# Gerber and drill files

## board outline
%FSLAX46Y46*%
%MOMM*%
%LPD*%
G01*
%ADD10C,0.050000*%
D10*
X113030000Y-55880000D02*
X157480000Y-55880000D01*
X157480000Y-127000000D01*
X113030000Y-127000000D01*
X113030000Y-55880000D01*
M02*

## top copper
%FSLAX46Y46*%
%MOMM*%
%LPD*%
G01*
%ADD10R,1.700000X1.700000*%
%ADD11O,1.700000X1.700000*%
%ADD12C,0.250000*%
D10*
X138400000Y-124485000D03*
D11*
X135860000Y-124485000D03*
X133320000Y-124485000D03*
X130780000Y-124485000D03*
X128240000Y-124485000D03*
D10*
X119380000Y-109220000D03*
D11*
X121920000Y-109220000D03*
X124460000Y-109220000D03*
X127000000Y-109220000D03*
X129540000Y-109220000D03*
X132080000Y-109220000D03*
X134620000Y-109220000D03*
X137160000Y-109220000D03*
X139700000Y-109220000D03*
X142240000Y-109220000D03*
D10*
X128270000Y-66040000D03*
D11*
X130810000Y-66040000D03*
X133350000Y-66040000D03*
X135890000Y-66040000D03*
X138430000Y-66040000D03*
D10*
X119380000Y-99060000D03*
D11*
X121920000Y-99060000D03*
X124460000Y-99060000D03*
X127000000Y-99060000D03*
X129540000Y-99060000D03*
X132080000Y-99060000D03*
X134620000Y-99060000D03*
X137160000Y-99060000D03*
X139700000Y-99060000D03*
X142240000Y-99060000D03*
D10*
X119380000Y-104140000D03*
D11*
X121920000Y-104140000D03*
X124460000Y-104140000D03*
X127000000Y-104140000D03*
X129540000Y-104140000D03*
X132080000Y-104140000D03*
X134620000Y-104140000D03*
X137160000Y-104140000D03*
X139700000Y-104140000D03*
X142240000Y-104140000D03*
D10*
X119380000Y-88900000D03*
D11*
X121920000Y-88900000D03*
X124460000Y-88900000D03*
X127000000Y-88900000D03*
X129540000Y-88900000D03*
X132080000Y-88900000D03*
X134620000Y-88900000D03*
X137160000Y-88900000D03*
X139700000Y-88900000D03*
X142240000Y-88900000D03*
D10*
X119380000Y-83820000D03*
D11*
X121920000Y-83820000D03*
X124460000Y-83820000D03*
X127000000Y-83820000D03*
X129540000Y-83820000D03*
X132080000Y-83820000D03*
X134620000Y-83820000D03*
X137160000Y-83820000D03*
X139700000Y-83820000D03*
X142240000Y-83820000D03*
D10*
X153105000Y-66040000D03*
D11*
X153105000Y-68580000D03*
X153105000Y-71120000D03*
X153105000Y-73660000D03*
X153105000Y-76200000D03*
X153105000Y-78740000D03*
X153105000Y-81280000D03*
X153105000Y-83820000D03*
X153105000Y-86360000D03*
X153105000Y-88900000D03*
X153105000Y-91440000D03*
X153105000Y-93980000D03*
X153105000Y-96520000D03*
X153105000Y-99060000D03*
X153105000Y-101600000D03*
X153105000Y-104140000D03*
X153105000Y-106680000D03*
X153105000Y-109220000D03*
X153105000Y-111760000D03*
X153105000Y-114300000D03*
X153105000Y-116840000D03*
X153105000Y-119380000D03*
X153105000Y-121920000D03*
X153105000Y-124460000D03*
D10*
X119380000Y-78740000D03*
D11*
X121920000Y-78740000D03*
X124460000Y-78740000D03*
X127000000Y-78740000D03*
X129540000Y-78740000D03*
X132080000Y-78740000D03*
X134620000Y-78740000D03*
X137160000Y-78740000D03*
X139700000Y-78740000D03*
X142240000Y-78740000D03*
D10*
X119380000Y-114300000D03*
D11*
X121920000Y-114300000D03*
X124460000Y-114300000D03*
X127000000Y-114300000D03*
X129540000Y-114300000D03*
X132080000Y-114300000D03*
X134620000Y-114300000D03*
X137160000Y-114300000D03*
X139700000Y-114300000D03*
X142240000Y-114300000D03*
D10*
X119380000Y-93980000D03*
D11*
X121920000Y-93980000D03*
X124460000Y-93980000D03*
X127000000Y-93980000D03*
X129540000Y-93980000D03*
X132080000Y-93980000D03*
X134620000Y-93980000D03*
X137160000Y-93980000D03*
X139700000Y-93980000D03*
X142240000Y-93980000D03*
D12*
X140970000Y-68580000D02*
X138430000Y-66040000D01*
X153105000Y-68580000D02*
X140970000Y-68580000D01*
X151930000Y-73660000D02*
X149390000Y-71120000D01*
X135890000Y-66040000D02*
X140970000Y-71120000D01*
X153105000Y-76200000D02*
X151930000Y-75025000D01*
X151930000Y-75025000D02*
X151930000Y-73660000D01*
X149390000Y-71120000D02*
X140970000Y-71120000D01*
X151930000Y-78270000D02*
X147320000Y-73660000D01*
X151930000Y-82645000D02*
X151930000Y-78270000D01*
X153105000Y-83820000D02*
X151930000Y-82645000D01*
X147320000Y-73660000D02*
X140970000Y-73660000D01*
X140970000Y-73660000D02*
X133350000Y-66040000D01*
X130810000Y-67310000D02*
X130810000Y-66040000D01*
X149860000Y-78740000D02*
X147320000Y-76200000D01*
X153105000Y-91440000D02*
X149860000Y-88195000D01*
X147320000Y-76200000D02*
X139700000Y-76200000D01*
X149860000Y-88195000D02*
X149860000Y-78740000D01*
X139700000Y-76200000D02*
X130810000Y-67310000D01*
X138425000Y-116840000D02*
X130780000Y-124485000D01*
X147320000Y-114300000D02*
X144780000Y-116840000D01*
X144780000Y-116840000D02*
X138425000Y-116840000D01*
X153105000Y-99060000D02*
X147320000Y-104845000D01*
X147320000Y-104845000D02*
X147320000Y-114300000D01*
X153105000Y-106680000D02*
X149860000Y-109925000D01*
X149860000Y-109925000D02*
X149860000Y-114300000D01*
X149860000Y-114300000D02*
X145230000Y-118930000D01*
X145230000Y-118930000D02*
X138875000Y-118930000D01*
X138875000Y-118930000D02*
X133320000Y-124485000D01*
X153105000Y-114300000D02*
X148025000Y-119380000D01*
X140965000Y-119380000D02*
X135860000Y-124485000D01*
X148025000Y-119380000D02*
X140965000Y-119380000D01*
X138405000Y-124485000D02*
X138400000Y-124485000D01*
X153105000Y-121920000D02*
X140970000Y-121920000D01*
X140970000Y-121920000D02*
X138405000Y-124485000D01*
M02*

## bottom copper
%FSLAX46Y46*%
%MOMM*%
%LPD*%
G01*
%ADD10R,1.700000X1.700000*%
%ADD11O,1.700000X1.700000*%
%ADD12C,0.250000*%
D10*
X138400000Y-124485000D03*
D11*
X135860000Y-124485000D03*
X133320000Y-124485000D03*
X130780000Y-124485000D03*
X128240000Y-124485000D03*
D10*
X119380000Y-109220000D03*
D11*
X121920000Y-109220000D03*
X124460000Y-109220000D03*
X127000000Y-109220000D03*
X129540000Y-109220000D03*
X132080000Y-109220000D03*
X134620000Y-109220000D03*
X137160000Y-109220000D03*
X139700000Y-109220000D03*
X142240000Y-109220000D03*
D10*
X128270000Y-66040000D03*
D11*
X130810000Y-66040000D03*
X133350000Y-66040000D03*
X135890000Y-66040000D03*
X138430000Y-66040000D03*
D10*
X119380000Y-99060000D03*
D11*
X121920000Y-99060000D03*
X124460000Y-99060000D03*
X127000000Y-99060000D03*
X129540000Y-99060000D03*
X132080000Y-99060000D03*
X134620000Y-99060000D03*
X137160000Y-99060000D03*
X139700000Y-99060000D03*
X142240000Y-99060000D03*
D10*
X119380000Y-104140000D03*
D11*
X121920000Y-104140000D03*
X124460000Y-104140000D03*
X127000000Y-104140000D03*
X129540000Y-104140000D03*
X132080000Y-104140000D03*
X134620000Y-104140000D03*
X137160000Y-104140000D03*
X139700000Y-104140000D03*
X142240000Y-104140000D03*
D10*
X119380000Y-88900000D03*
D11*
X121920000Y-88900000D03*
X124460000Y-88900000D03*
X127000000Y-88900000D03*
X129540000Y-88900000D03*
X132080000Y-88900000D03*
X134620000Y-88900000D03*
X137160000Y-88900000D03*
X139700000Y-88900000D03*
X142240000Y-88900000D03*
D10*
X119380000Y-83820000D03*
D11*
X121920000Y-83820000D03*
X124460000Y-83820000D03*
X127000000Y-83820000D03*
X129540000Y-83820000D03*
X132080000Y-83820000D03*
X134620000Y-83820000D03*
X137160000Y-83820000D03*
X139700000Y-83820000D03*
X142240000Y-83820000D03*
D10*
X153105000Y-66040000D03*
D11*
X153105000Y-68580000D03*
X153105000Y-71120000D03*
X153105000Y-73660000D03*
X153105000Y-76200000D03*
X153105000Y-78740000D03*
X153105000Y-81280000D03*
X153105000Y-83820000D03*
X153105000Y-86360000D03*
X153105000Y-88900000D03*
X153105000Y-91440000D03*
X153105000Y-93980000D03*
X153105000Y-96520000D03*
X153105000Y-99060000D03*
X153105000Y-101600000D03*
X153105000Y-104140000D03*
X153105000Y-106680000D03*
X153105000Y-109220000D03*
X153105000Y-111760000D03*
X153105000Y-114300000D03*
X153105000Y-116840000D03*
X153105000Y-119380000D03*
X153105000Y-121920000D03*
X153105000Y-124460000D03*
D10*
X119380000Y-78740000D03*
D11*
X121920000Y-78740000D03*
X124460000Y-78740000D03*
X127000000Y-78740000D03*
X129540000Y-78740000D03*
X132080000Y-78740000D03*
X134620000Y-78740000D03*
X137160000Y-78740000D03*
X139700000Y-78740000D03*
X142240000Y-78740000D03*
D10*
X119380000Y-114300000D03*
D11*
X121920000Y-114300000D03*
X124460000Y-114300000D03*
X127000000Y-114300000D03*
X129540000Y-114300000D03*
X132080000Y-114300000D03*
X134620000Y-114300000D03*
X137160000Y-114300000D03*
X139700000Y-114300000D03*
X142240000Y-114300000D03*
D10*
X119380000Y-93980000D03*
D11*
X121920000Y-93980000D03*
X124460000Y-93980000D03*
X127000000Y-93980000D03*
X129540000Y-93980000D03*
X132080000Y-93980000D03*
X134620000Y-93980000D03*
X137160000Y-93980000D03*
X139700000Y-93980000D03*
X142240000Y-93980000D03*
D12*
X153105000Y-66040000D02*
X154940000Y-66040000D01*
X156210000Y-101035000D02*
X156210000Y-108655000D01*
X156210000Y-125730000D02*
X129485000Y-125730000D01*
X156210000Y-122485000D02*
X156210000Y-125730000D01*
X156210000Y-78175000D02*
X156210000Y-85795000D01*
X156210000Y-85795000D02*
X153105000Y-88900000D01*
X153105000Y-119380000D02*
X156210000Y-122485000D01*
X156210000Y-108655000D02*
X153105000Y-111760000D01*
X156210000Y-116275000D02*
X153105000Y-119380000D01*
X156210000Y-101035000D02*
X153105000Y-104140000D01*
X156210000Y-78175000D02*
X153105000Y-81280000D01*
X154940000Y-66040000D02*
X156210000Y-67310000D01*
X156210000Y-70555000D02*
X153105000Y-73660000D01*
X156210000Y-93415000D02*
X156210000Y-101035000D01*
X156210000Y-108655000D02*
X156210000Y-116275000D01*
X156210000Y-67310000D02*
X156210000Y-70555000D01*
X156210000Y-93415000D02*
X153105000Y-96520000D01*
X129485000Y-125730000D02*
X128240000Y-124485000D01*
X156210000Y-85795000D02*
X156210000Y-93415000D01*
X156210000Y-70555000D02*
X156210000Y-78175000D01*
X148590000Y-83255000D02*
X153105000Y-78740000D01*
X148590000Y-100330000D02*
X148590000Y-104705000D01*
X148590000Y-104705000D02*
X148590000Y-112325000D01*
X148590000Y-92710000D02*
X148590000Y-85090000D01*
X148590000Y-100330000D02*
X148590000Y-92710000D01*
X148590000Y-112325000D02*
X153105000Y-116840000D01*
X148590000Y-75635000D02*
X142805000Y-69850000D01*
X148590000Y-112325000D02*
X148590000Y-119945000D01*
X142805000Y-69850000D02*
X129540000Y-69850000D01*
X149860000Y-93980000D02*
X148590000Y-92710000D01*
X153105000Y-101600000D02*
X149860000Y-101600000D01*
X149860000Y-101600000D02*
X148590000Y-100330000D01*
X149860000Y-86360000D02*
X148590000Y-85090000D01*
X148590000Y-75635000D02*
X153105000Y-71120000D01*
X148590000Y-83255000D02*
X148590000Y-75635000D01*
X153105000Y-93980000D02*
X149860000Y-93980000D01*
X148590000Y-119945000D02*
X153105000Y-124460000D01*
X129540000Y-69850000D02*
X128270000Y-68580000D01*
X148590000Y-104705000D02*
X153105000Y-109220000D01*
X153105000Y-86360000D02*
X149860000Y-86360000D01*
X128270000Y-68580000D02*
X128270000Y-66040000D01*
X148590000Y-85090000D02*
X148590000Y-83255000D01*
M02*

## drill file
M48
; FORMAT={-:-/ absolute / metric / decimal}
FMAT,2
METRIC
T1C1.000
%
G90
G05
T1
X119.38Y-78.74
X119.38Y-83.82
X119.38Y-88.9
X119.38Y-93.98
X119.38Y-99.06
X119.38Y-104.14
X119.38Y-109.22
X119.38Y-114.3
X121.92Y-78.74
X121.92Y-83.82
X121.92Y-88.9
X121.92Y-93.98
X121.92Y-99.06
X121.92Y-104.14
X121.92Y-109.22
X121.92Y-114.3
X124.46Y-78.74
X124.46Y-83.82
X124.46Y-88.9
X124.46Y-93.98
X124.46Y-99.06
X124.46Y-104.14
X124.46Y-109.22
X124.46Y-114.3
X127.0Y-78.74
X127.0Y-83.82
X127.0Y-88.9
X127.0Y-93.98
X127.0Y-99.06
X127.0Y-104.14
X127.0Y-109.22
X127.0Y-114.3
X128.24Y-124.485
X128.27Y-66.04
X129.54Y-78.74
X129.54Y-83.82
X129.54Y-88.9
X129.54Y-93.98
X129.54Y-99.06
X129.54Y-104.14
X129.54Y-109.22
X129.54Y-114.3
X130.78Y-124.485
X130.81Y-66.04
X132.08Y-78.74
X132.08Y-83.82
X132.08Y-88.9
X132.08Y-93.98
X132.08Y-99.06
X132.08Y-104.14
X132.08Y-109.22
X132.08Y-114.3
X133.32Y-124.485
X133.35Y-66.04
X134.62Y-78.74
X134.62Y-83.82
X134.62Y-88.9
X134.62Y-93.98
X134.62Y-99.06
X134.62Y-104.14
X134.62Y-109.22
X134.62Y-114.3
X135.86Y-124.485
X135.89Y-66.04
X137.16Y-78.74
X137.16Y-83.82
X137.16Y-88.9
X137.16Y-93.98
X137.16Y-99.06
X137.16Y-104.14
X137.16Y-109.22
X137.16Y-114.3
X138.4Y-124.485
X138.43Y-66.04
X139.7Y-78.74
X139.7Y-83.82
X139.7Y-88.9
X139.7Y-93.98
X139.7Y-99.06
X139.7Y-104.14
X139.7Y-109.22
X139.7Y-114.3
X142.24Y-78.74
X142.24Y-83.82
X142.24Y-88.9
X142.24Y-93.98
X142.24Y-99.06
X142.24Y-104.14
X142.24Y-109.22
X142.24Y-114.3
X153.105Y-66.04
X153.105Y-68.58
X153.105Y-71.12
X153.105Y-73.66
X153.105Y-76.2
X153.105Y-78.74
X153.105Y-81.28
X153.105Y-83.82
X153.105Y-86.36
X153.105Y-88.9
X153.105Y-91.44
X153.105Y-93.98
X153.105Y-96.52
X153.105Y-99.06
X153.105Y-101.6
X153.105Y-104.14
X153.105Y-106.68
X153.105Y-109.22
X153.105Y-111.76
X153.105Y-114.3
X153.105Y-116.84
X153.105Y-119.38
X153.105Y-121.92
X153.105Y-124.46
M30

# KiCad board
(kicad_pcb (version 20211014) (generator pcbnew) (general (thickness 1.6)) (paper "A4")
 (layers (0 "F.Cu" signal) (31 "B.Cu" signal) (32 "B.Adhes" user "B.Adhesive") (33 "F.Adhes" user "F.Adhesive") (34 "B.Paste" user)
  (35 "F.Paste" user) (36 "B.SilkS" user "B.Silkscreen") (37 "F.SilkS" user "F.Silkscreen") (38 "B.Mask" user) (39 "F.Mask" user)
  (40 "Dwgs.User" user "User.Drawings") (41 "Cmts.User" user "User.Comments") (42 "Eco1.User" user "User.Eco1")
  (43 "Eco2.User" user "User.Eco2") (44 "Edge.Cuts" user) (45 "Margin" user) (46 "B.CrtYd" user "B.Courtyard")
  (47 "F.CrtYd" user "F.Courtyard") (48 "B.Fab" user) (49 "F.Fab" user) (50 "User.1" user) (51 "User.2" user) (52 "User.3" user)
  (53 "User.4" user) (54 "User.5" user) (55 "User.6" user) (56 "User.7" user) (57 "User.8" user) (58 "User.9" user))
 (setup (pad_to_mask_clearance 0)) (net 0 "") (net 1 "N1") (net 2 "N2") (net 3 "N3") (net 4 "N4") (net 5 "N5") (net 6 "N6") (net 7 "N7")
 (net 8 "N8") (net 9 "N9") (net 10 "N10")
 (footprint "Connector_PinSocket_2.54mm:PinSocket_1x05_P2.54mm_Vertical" (layer "F.Cu") (at 138.4 124.485 -90)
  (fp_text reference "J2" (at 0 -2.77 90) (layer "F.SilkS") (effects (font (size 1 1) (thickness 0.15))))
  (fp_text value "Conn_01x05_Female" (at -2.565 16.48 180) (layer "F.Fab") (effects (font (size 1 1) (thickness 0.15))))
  (pad "1" thru_hole rect (at 0 0 270) (size 1.7 1.7) (drill 1) (layers *.Cu *.Mask) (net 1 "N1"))
  (pad "2" thru_hole oval (at 0 2.54 270) (size 1.7 1.7) (drill 1) (layers *.Cu *.Mask) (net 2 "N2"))
  (pad "3" thru_hole oval (at 0 5.08 270) (size 1.7 1.7) (drill 1) (layers *.Cu *.Mask) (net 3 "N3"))
  (pad "4" thru_hole oval (at 0 7.62 270) (size 1.7 1.7) (drill 1) (layers *.Cu *.Mask) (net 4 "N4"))
  (pad "5" thru_hole oval (at 0 10.16 270) (size 1.7 1.7) (drill 1) (layers *.Cu *.Mask) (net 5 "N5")))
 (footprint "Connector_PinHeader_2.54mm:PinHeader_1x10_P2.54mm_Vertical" (layer "F.Cu") (at 119.38 109.22 90)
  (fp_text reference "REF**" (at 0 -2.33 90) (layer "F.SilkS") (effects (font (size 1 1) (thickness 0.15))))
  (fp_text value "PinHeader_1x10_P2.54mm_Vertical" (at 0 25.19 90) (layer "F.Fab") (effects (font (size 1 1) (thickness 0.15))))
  (pad "1" thru_hole rect (at 0 0 90) (size 1.7 1.7) (drill 1) (layers *.Cu *.Mask))
  (pad "2" thru_hole oval (at 0 2.54 90) (size 1.7 1.7) (drill 1) (layers *.Cu *.Mask))
  (pad "3" thru_hole oval (at 0 5.08 90) (size 1.7 1.7) (drill 1) (layers *.Cu *.Mask))
  (pad "4" thru_hole oval (at 0 7.62 90) (size 1.7 1.7) (drill 1) (layers *.Cu *.Mask))
  (pad "5" thru_hole oval (at 0 10.16 90) (size 1.7 1.7) (drill 1) (layers *.Cu *.Mask))
  (pad "6" thru_hole oval (at 0 12.7 90) (size 1.7 1.7) (drill 1) (layers *.Cu *.Mask))
  (pad "7" thru_hole oval (at 0 15.24 90) (size 1.7 1.7) (drill 1) (layers *.Cu *.Mask))
  (pad "8" thru_hole oval (at 0 17.78 90) (size 1.7 1.7) (drill 1) (layers *.Cu *.Mask))
  (pad "9" thru_hole oval (at 0 20.32 90) (size 1.7 1.7) (drill 1) (layers *.Cu *.Mask))
  (pad "10" thru_hole oval (at 0 22.86 90) (size 1.7 1.7) (drill 1) (layers *.Cu *.Mask)))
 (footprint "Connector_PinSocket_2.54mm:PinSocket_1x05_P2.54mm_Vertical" (layer "F.Cu") (at 128.27 66.04 90)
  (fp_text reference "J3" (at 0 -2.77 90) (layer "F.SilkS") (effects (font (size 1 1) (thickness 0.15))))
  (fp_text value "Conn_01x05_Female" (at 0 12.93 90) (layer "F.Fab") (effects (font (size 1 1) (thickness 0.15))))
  (pad "1" thru_hole rect (at 0 0 90) (size 1.7 1.7) (drill 1) (layers *.Cu *.Mask) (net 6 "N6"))
  (pad "2" thru_hole oval (at 0 2.54 90) (size 1.7 1.7) (drill 1) (layers *.Cu *.Mask) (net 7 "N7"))
  (pad "3" thru_hole oval (at 0 5.08 90) (size 1.7 1.7) (drill 1) (layers *.Cu *.Mask) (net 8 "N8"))
  (pad "4" thru_hole oval (at 0 7.62 90) (size 1.7 1.7) (drill 1) (layers *.Cu *.Mask) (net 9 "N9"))
  (pad "5" thru_hole oval (at 0 10.16 90) (size 1.7 1.7) (drill 1) (layers *.Cu *.Mask) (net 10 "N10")))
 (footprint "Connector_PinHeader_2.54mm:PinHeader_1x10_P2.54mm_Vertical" (layer "F.Cu") (at 119.38 99.06 90)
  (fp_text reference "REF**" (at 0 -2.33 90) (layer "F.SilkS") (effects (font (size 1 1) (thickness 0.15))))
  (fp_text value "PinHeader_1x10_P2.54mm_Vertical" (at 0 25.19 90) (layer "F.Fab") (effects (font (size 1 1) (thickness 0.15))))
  (pad "1" thru_hole rect (at 0 0 90) (size 1.7 1.7) (drill 1) (layers *.Cu *.Mask))
  (pad "2" thru_hole oval (at 0 2.54 90) (size 1.7 1.7) (drill 1) (layers *.Cu *.Mask))
  (pad "3" thru_hole oval (at 0 5.08 90) (size 1.7 1.7) (drill 1) (layers *.Cu *.Mask))
  (pad "4" thru_hole oval (at 0 7.62 90) (size 1.7 1.7) (drill 1) (layers *.Cu *.Mask))
  (pad "5" thru_hole oval (at 0 10.16 90) (size 1.7 1.7) (drill 1) (layers *.Cu *.Mask))
  (pad "6" thru_hole oval (at 0 12.7 90) (size 1.7 1.7) (drill 1) (layers *.Cu *.Mask))
  (pad "7" thru_hole oval (at 0 15.24 90) (size 1.7 1.7) (drill 1) (layers *.Cu *.Mask))
  (pad "8" thru_hole oval (at 0 17.78 90) (size 1.7 1.7) (drill 1) (layers *.Cu *.Mask))
  (pad "9" thru_hole oval (at 0 20.32 90) (size 1.7 1.7) (drill 1) (layers *.Cu *.Mask))
  (pad "10" thru_hole oval (at 0 22.86 90) (size 1.7 1.7) (drill 1) (layers *.Cu *.Mask)))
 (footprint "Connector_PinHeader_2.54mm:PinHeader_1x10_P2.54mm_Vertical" (layer "F.Cu") (at 119.38 104.14 90)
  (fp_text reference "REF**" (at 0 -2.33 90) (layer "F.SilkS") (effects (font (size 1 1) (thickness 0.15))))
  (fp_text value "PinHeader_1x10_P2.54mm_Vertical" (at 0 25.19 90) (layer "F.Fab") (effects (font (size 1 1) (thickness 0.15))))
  (pad "1" thru_hole rect (at 0 0 90) (size 1.7 1.7) (drill 1) (layers *.Cu *.Mask))
  (pad "2" thru_hole oval (at 0 2.54 90) (size 1.7 1.7) (drill 1) (layers *.Cu *.Mask))
  (pad "3" thru_hole oval (at 0 5.08 90) (size 1.7 1.7) (drill 1) (layers *.Cu *.Mask))
  (pad "4" thru_hole oval (at 0 7.62 90) (size 1.7 1.7) (drill 1) (layers *.Cu *.Mask))
  (pad "5" thru_hole oval (at 0 10.16 90) (size 1.7 1.7) (drill 1) (layers *.Cu *.Mask))
  (pad "6" thru_hole oval (at 0 12.7 90) (size 1.7 1.7) (drill 1) (layers *.Cu *.Mask))
  (pad "7" thru_hole oval (at 0 15.24 90) (size 1.7 1.7) (drill 1) (layers *.Cu *.Mask))
  (pad "8" thru_hole oval (at 0 17.78 90) (size 1.7 1.7) (drill 1) (layers *.Cu *.Mask))
  (pad "9" thru_hole oval (at 0 20.32 90) (size 1.7 1.7) (drill 1) (layers *.Cu *.Mask))
  (pad "10" thru_hole oval (at 0 22.86 90) (size 1.7 1.7) (drill 1) (layers *.Cu *.Mask)))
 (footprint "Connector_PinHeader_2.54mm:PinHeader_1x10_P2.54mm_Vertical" (layer "F.Cu") (at 119.38 88.9 90)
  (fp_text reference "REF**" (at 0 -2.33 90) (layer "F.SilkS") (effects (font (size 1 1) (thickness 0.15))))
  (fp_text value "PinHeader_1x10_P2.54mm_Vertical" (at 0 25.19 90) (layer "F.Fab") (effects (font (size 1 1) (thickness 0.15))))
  (pad "1" thru_hole rect (at 0 0 90) (size 1.7 1.7) (drill 1) (layers *.Cu *.Mask))
  (pad "2" thru_hole oval (at 0 2.54 90) (size 1.7 1.7) (drill 1) (layers *.Cu *.Mask))
  (pad "3" thru_hole oval (at 0 5.08 90) (size 1.7 1.7) (drill 1) (layers *.Cu *.Mask))
  (pad "4" thru_hole oval (at 0 7.62 90) (size 1.7 1.7) (drill 1) (layers *.Cu *.Mask))
  (pad "5" thru_hole oval (at 0 10.16 90) (size 1.7 1.7) (drill 1) (layers *.Cu *.Mask))
  (pad "6" thru_hole oval (at 0 12.7 90) (size 1.7 1.7) (drill 1) (layers *.Cu *.Mask))
  (pad "7" thru_hole oval (at 0 15.24 90) (size 1.7 1.7) (drill 1) (layers *.Cu *.Mask))
  (pad "8" thru_hole oval (at 0 17.78 90) (size 1.7 1.7) (drill 1) (layers *.Cu *.Mask))
  (pad "9" thru_hole oval (at 0 20.32 90) (size 1.7 1.7) (drill 1) (layers *.Cu *.Mask))
  (pad "10" thru_hole oval (at 0 22.86 90) (size 1.7 1.7) (drill 1) (layers *.Cu *.Mask)))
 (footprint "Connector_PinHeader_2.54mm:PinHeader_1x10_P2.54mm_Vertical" (layer "F.Cu") (at 119.38 83.82 90)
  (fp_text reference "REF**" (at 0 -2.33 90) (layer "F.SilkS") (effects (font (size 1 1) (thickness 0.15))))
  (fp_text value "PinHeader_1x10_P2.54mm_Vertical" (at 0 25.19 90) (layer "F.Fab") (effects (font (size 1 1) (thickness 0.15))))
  (pad "1" thru_hole rect (at 0 0 90) (size 1.7 1.7) (drill 1) (layers *.Cu *.Mask))
  (pad "2" thru_hole oval (at 0 2.54 90) (size 1.7 1.7) (drill 1) (layers *.Cu *.Mask))
  (pad "3" thru_hole oval (at 0 5.08 90) (size 1.7 1.7) (drill 1) (layers *.Cu *.Mask))
  (pad "4" thru_hole oval (at 0 7.62 90) (size 1.7 1.7) (drill 1) (layers *.Cu *.Mask))
  (pad "5" thru_hole oval (at 0 10.16 90) (size 1.7 1.7) (drill 1) (layers *.Cu *.Mask))
  (pad "6" thru_hole oval (at 0 12.7 90) (size 1.7 1.7) (drill 1) (layers *.Cu *.Mask))
  (pad "7" thru_hole oval (at 0 15.24 90) (size 1.7 1.7) (drill 1) (layers *.Cu *.Mask))
  (pad "8" thru_hole oval (at 0 17.78 90) (size 1.7 1.7) (drill 1) (layers *.Cu *.Mask))
  (pad "9" thru_hole oval (at 0 20.32 90) (size 1.7 1.7) (drill 1) (layers *.Cu *.Mask))
  (pad "10" thru_hole oval (at 0 22.86 90) (size 1.7 1.7) (drill 1) (layers *.Cu *.Mask)))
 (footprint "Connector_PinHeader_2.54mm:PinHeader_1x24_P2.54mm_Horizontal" (layer "F.Cu") (at 153.105 66.04)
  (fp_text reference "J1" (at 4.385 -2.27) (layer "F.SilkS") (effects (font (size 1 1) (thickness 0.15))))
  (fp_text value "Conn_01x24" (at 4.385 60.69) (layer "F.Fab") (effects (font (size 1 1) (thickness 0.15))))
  (pad "1" thru_hole rect (at 0 0) (size 1.7 1.7) (drill 1) (layers *.Cu *.Mask) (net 5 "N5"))
  (pad "2" thru_hole oval (at 0 2.54) (size 1.7 1.7) (drill 1) (layers *.Cu *.Mask) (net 10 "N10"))
  (pad "3" thru_hole oval (at 0 5.08) (size 1.7 1.7) (drill 1) (layers *.Cu *.Mask) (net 6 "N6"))
  (pad "4" thru_hole oval (at 0 7.62) (size 1.7 1.7) (drill 1) (layers *.Cu *.Mask) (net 5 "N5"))
  (pad "5" thru_hole oval (at 0 10.16) (size 1.7 1.7) (drill 1) (layers *.Cu *.Mask) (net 9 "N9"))
  (pad "6" thru_hole oval (at 0 12.7) (size 1.7 1.7) (drill 1) (layers *.Cu *.Mask) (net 6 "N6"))
  (pad "7" thru_hole oval (at 0 15.24) (size 1.7 1.7) (drill 1) (layers *.Cu *.Mask) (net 5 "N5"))
  (pad "8" thru_hole oval (at 0 17.78) (size 1.7 1.7) (drill 1) (layers *.Cu *.Mask) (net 8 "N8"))
  (pad "9" thru_hole oval (at 0 20.32) (size 1.7 1.7) (drill 1) (layers *.Cu *.Mask) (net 6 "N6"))
  (pad "10" thru_hole oval (at 0 22.86) (size 1.7 1.7) (drill 1) (layers *.Cu *.Mask) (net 5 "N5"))
  (pad "11" thru_hole oval (at 0 25.4) (size 1.7 1.7) (drill 1) (layers *.Cu *.Mask) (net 7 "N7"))
  (pad "12" thru_hole oval (at 0 27.94) (size 1.7 1.7) (drill 1) (layers *.Cu *.Mask) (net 6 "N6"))
  (pad "13" thru_hole oval (at 0 30.48) (size 1.7 1.7) (drill 1) (layers *.Cu *.Mask) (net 5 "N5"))
  (pad "14" thru_hole oval (at 0 33.02) (size 1.7 1.7) (drill 1) (layers *.Cu *.Mask) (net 4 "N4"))
  (pad "15" thru_hole oval (at 0 35.56) (size 1.7 1.7) (drill 1) (layers *.Cu *.Mask) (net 6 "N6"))
  (pad "16" thru_hole oval (at 0 38.1) (size 1.7 1.7) (drill 1) (layers *.Cu *.Mask) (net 5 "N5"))
  (pad "17" thru_hole oval (at 0 40.64) (size 1.7 1.7) (drill 1) (layers *.Cu *.Mask) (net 3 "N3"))
  (pad "18" thru_hole oval (at 0 43.18) (size 1.7 1.7) (drill 1) (layers *.Cu *.Mask) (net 6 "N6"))
  (pad "19" thru_hole oval (at 0 45.72) (size 1.7 1.7) (drill 1) (layers *.Cu *.Mask) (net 5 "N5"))
  (pad "20" thru_hole oval (at 0 48.26) (size 1.7 1.7) (drill 1) (layers *.Cu *.Mask) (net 2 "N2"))
  (pad "21" thru_hole oval (at 0 50.8) (size 1.7 1.7) (drill 1) (layers *.Cu *.Mask) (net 6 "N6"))
  (pad "22" thru_hole oval (at 0 53.34) (size 1.7 1.7) (drill 1) (layers *.Cu *.Mask) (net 5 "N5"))
  (pad "23" thru_hole oval (at 0 55.88) (size 1.7 1.7) (drill 1) (layers *.Cu *.Mask) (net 1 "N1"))
  (pad "24" thru_hole oval (at 0 58.42) (size 1.7 1.7) (drill 1) (layers *.Cu *.Mask) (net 6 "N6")))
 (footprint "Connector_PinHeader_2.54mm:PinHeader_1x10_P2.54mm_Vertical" (layer "F.Cu") (at 119.38 78.74 90)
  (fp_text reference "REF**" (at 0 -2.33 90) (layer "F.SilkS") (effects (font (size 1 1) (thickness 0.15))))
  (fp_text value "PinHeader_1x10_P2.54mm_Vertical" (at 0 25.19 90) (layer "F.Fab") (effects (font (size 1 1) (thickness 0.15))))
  (pad "1" thru_hole rect (at 0 0 90) (size 1.7 1.7) (drill 1) (layers *.Cu *.Mask))
  (pad "2" thru_hole oval (at 0 2.54 90) (size 1.7 1.7) (drill 1) (layers *.Cu *.Mask))
  (pad "3" thru_hole oval (at 0 5.08 90) (size 1.7 1.7) (drill 1) (layers *.Cu *.Mask))
  (pad "4" thru_hole oval (at 0 7.62 90) (size 1.7 1.7) (drill 1) (layers *.Cu *.Mask))
  (pad "5" thru_hole oval (at 0 10.16 90) (size 1.7 1.7) (drill 1) (layers *.Cu *.Mask))
  (pad "6" thru_hole oval (at 0 12.7 90) (size 1.7 1.7) (drill 1) (layers *.Cu *.Mask))
  (pad "7" thru_hole oval (at 0 15.24 90) (size 1.7 1.7) (drill 1) (layers *.Cu *.Mask))
  (pad "8" thru_hole oval (at 0 17.78 90) (size 1.7 1.7) (drill 1) (layers *.Cu *.Mask))
  (pad "9" thru_hole oval (at 0 20.32 90) (size 1.7 1.7) (drill 1) (layers *.Cu *.Mask))
  (pad "10" thru_hole oval (at 0 22.86 90) (size 1.7 1.7) (drill 1) (layers *.Cu *.Mask)))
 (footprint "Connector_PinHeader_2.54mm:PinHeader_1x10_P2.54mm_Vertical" (layer "F.Cu") (at 119.38 114.3 90)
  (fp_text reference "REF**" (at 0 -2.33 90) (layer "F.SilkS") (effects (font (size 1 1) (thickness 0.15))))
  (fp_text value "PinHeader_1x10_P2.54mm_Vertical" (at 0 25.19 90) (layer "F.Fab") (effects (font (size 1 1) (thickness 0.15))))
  (pad "1" thru_hole rect (at 0 0 90) (size 1.7 1.7) (drill 1) (layers *.Cu *.Mask))
  (pad "2" thru_hole oval (at 0 2.54 90) (size 1.7 1.7) (drill 1) (layers *.Cu *.Mask))
  (pad "3" thru_hole oval (at 0 5.08 90) (size 1.7 1.7) (drill 1) (layers *.Cu *.Mask))
  (pad "4" thru_hole oval (at 0 7.62 90) (size 1.7 1.7) (drill 1) (layers *.Cu *.Mask))
  (pad "5" thru_hole oval (at 0 10.16 90) (size 1.7 1.7) (drill 1) (layers *.Cu *.Mask))
  (pad "6" thru_hole oval (at 0 12.7 90) (size 1.7 1.7) (drill 1) (layers *.Cu *.Mask))
  (pad "7" thru_hole oval (at 0 15.24 90) (size 1.7 1.7) (drill 1) (layers *.Cu *.Mask))
  (pad "8" thru_hole oval (at 0 17.78 90) (size 1.7 1.7) (drill 1) (layers *.Cu *.Mask))
  (pad "9" thru_hole oval (at 0 20.32 90) (size 1.7 1.7) (drill 1) (layers *.Cu *.Mask))
  (pad "10" thru_hole oval (at 0 22.86 90) (size 1.7 1.7) (drill 1) (layers *.Cu *.Mask)))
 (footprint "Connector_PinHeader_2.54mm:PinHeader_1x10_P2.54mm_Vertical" (layer "F.Cu") (at 119.38 93.98 90)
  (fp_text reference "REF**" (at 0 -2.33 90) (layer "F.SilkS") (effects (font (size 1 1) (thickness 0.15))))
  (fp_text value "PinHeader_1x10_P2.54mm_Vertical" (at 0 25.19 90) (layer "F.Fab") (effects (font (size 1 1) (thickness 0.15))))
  (pad "1" thru_hole rect (at 0 0 90) (size 1.7 1.7) (drill 1) (layers *.Cu *.Mask))
  (pad "2" thru_hole oval (at 0 2.54 90) (size 1.7 1.7) (drill 1) (layers *.Cu *.Mask))
  (pad "3" thru_hole oval (at 0 5.08 90) (size 1.7 1.7) (drill 1) (layers *.Cu *.Mask))
  (pad "4" thru_hole oval (at 0 7.62 90) (size 1.7 1.7) (drill 1) (layers *.Cu *.Mask))
  (pad "5" thru_hole oval (at 0 10.16 90) (size 1.7 1.7) (drill 1) (layers *.Cu *.Mask))
  (pad "6" thru_hole oval (at 0 12.7 90) (size 1.7 1.7) (drill 1) (layers *.Cu *.Mask))
  (pad "7" thru_hole oval (at 0 15.24 90) (size 1.7 1.7) (drill 1) (layers *.Cu *.Mask))
  (pad "8" thru_hole oval (at 0 17.78 90) (size 1.7 1.7) (drill 1) (layers *.Cu *.Mask))
  (pad "9" thru_hole oval (at 0 20.32 90) (size 1.7 1.7) (drill 1) (layers *.Cu *.Mask))
  (pad "10" thru_hole oval (at 0 22.86 90) (size 1.7 1.7) (drill 1) (layers *.Cu *.Mask)))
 (gr_rect (start 157.48 127) (end 113.03 55.88) (layer "Edge.Cuts") (width 0.05) (fill none))
 (segment (start 153.105 66.04) (end 154.94 66.04) (width 0.25) (layer "B.Cu") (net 5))
 (segment (start 156.21 101.035) (end 156.21 108.655) (width 0.25) (layer "B.Cu") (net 5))
 (segment (start 156.21 125.73) (end 129.485 125.73) (width 0.25) (layer "B.Cu") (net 5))
 (segment (start 156.21 122.485) (end 156.21 125.73) (width 0.25) (layer "B.Cu") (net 5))
 (segment (start 156.21 78.175) (end 156.21 85.795) (width 0.25) (layer "B.Cu") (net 5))
 (segment (start 156.21 85.795) (end 153.105 88.9) (width 0.25) (layer "B.Cu") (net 5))
 (segment (start 153.105 119.38) (end 156.21 122.485) (width 0.25) (layer "B.Cu") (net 5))
 (segment (start 156.21 108.655) (end 153.105 111.76) (width 0.25) (layer "B.Cu") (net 5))
 (segment (start 156.21 116.275) (end 153.105 119.38) (width 0.25) (layer "B.Cu") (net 5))
 (segment (start 156.21 101.035) (end 153.105 104.14) (width 0.25) (layer "B.Cu") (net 5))
 (segment (start 156.21 78.175) (end 153.105 81.28) (width 0.25) (layer "B.Cu") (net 5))
 (segment (start 154.94 66.04) (end 156.21 67.31) (width 0.25) (layer "B.Cu") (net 5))
 (segment (start 156.21 70.555) (end 153.105 73.66) (width 0.25) (layer "B.Cu") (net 5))
 (segment (start 156.21 93.415) (end 156.21 101.035) (width 0.25) (layer "B.Cu") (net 5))
 (segment (start 156.21 108.655) (end 156.21 116.275) (width 0.25) (layer "B.Cu") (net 5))
 (segment (start 156.21 67.31) (end 156.21 70.555) (width 0.25) (layer "B.Cu") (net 5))
 (segment (start 156.21 93.415) (end 153.105 96.52) (width 0.25) (layer "B.Cu") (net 5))
 (segment (start 129.485 125.73) (end 128.24 124.485) (width 0.25) (layer "B.Cu") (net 5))
 (segment (start 156.21 85.795) (end 156.21 93.415) (width 0.25) (layer "B.Cu") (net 5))
 (segment (start 156.21 70.555) (end 156.21 78.175) (width 0.25) (layer "B.Cu") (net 5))
 (segment (start 140.97 68.58) (end 138.43 66.04) (width 0.25) (layer "F.Cu") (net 10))
 (segment (start 153.105 68.58) (end 140.97 68.58) (width 0.25) (layer "F.Cu") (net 10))
 (segment (start 151.93 73.66) (end 149.39 71.12) (width 0.25) (layer "F.Cu") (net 9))
 (segment (start 135.89 66.04) (end 140.97 71.12) (width 0.25) (layer "F.Cu") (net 9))
 (segment (start 153.105 76.2) (end 151.93 75.025) (width 0.25) (layer "F.Cu") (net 9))
 (segment (start 151.93 75.025) (end 151.93 73.66) (width 0.25) (layer "F.Cu") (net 9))
 (segment (start 149.39 71.12) (end 140.97 71.12) (width 0.25) (layer "F.Cu") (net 9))
 (segment (start 151.93 78.27) (end 147.32 73.66) (width 0.25) (layer "F.Cu") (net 8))
 (segment (start 151.93 82.645) (end 151.93 78.27) (width 0.25) (layer "F.Cu") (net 8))
 (segment (start 153.105 83.82) (end 151.93 82.645) (width 0.25) (layer "F.Cu") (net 8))
 (segment (start 147.32 73.66) (end 140.97 73.66) (width 0.25) (layer "F.Cu") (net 8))
 (segment (start 140.97 73.66) (end 133.35 66.04) (width 0.25) (layer "F.Cu") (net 8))
 (segment (start 130.81 67.31) (end 130.81 66.04) (width 0.25) (layer "F.Cu") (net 7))
 (segment (start 149.86 78.74) (end 147.32 76.2) (width 0.25) (layer "F.Cu") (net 7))
 (segment (start 153.105 91.44) (end 149.86 88.195) (width 0.25) (layer "F.Cu") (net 7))
 (segment (start 147.32 76.2) (end 139.7 76.2) (width 0.25) (layer "F.Cu") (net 7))
 (segment (start 149.86 88.195) (end 149.86 78.74) (width 0.25) (layer "F.Cu") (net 7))
 (segment (start 139.7 76.2) (end 130.81 67.31) (width 0.25) (layer "F.Cu") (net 7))
 (segment (start 148.59 83.255) (end 153.105 78.74) (width 0.25) (layer "B.Cu") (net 6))
 (segment (start 148.59 100.33) (end 148.59 104.705) (width 0.25) (layer "B.Cu") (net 6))
 (segment (start 148.59 104.705) (end 148.59 112.325) (width 0.25) (layer "B.Cu") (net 6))
 (segment (start 148.59 92.71) (end 148.59 85.09) (width 0.25) (layer "B.Cu") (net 6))
 (segment (start 148.59 100.33) (end 148.59 92.71) (width 0.25) (layer "B.Cu") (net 6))
 (segment (start 148.59 112.325) (end 153.105 116.84) (width 0.25) (layer "B.Cu") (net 6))
 (segment (start 148.59 75.635) (end 142.805 69.85) (width 0.25) (layer "B.Cu") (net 6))
 (segment (start 148.59 112.325) (end 148.59 119.945) (width 0.25) (layer "B.Cu") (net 6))
 (segment (start 142.805 69.85) (end 129.54 69.85) (width 0.25) (layer "B.Cu") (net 6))
 (segment (start 149.86 93.98) (end 148.59 92.71) (width 0.25) (layer "B.Cu") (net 6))
 (segment (start 153.105 101.6) (end 149.86 101.6) (width 0.25) (layer "B.Cu") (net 6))
 (segment (start 149.86 101.6) (end 148.59 100.33) (width 0.25) (layer "B.Cu") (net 6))
 (segment (start 149.86 86.36) (end 148.59 85.09) (width 0.25) (layer "B.Cu") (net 6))
 (segment (start 148.59 75.635) (end 153.105 71.12) (width 0.25) (layer "B.Cu") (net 6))
 (segment (start 148.59 83.255) (end 148.59 75.635) (width 0.25) (layer "B.Cu") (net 6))
 (segment (start 153.105 93.98) (end 149.86 93.98) (width 0.25) (layer "B.Cu") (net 6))
 (segment (start 148.59 119.945) (end 153.105 124.46) (width 0.25) (layer "B.Cu") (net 6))
 (segment (start 129.54 69.85) (end 128.27 68.58) (width 0.25) (layer "B.Cu") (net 6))
 (segment (start 148.59 104.705) (end 153.105 109.22) (width 0.25) (layer "B.Cu") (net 6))
 (segment (start 153.105 86.36) (end 149.86 86.36) (width 0.25) (layer "B.Cu") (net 6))
 (segment (start 128.27 68.58) (end 128.27 66.04) (width 0.25) (layer "B.Cu") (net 6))
 (segment (start 148.59 85.09) (end 148.59 83.255) (width 0.25) (layer "B.Cu") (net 6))
 (segment (start 138.425 116.84) (end 130.78 124.485) (width 0.25) (layer "F.Cu") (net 4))
 (segment (start 147.32 114.3) (end 144.78 116.84) (width 0.25) (layer "F.Cu") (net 4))
 (segment (start 144.78 116.84) (end 138.425 116.84) (width 0.25) (layer "F.Cu") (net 4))
 (segment (start 153.105 99.06) (end 147.32 104.845) (width 0.25) (layer "F.Cu") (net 4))
 (segment (start 147.32 104.845) (end 147.32 114.3) (width 0.25) (layer "F.Cu") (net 4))
 (segment (start 153.105 106.68) (end 149.86 109.925) (width 0.25) (layer "F.Cu") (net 3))
 (segment (start 149.86 109.925) (end 149.86 114.3) (width 0.25) (layer "F.Cu") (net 3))
 (segment (start 149.86 114.3) (end 145.23 118.93) (width 0.25) (layer "F.Cu") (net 3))
 (segment (start 145.23 118.93) (end 138.875 118.93) (width 0.25) (layer "F.Cu") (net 3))
 (segment (start 138.875 118.93) (end 133.32 124.485) (width 0.25) (layer "F.Cu") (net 3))
 (segment (start 153.105 114.3) (end 148.025 119.38) (width 0.25) (layer "F.Cu") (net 2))
 (segment (start 140.965 119.38) (end 135.86 124.485) (width 0.25) (layer "F.Cu") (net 2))
 (segment (start 148.025 119.38) (end 140.965 119.38) (width 0.25) (layer "F.Cu") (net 2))
 (segment (start 138.405 124.485) (end 138.4 124.485) (width 0.25) (layer "F.Cu") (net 1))
 (segment (start 153.105 121.92) (end 140.97 121.92) (width 0.25) (layer "F.Cu") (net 1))
 (segment (start 140.97 121.92) (end 138.405 124.485) (width 0.25) (layer "F.Cu") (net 1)))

